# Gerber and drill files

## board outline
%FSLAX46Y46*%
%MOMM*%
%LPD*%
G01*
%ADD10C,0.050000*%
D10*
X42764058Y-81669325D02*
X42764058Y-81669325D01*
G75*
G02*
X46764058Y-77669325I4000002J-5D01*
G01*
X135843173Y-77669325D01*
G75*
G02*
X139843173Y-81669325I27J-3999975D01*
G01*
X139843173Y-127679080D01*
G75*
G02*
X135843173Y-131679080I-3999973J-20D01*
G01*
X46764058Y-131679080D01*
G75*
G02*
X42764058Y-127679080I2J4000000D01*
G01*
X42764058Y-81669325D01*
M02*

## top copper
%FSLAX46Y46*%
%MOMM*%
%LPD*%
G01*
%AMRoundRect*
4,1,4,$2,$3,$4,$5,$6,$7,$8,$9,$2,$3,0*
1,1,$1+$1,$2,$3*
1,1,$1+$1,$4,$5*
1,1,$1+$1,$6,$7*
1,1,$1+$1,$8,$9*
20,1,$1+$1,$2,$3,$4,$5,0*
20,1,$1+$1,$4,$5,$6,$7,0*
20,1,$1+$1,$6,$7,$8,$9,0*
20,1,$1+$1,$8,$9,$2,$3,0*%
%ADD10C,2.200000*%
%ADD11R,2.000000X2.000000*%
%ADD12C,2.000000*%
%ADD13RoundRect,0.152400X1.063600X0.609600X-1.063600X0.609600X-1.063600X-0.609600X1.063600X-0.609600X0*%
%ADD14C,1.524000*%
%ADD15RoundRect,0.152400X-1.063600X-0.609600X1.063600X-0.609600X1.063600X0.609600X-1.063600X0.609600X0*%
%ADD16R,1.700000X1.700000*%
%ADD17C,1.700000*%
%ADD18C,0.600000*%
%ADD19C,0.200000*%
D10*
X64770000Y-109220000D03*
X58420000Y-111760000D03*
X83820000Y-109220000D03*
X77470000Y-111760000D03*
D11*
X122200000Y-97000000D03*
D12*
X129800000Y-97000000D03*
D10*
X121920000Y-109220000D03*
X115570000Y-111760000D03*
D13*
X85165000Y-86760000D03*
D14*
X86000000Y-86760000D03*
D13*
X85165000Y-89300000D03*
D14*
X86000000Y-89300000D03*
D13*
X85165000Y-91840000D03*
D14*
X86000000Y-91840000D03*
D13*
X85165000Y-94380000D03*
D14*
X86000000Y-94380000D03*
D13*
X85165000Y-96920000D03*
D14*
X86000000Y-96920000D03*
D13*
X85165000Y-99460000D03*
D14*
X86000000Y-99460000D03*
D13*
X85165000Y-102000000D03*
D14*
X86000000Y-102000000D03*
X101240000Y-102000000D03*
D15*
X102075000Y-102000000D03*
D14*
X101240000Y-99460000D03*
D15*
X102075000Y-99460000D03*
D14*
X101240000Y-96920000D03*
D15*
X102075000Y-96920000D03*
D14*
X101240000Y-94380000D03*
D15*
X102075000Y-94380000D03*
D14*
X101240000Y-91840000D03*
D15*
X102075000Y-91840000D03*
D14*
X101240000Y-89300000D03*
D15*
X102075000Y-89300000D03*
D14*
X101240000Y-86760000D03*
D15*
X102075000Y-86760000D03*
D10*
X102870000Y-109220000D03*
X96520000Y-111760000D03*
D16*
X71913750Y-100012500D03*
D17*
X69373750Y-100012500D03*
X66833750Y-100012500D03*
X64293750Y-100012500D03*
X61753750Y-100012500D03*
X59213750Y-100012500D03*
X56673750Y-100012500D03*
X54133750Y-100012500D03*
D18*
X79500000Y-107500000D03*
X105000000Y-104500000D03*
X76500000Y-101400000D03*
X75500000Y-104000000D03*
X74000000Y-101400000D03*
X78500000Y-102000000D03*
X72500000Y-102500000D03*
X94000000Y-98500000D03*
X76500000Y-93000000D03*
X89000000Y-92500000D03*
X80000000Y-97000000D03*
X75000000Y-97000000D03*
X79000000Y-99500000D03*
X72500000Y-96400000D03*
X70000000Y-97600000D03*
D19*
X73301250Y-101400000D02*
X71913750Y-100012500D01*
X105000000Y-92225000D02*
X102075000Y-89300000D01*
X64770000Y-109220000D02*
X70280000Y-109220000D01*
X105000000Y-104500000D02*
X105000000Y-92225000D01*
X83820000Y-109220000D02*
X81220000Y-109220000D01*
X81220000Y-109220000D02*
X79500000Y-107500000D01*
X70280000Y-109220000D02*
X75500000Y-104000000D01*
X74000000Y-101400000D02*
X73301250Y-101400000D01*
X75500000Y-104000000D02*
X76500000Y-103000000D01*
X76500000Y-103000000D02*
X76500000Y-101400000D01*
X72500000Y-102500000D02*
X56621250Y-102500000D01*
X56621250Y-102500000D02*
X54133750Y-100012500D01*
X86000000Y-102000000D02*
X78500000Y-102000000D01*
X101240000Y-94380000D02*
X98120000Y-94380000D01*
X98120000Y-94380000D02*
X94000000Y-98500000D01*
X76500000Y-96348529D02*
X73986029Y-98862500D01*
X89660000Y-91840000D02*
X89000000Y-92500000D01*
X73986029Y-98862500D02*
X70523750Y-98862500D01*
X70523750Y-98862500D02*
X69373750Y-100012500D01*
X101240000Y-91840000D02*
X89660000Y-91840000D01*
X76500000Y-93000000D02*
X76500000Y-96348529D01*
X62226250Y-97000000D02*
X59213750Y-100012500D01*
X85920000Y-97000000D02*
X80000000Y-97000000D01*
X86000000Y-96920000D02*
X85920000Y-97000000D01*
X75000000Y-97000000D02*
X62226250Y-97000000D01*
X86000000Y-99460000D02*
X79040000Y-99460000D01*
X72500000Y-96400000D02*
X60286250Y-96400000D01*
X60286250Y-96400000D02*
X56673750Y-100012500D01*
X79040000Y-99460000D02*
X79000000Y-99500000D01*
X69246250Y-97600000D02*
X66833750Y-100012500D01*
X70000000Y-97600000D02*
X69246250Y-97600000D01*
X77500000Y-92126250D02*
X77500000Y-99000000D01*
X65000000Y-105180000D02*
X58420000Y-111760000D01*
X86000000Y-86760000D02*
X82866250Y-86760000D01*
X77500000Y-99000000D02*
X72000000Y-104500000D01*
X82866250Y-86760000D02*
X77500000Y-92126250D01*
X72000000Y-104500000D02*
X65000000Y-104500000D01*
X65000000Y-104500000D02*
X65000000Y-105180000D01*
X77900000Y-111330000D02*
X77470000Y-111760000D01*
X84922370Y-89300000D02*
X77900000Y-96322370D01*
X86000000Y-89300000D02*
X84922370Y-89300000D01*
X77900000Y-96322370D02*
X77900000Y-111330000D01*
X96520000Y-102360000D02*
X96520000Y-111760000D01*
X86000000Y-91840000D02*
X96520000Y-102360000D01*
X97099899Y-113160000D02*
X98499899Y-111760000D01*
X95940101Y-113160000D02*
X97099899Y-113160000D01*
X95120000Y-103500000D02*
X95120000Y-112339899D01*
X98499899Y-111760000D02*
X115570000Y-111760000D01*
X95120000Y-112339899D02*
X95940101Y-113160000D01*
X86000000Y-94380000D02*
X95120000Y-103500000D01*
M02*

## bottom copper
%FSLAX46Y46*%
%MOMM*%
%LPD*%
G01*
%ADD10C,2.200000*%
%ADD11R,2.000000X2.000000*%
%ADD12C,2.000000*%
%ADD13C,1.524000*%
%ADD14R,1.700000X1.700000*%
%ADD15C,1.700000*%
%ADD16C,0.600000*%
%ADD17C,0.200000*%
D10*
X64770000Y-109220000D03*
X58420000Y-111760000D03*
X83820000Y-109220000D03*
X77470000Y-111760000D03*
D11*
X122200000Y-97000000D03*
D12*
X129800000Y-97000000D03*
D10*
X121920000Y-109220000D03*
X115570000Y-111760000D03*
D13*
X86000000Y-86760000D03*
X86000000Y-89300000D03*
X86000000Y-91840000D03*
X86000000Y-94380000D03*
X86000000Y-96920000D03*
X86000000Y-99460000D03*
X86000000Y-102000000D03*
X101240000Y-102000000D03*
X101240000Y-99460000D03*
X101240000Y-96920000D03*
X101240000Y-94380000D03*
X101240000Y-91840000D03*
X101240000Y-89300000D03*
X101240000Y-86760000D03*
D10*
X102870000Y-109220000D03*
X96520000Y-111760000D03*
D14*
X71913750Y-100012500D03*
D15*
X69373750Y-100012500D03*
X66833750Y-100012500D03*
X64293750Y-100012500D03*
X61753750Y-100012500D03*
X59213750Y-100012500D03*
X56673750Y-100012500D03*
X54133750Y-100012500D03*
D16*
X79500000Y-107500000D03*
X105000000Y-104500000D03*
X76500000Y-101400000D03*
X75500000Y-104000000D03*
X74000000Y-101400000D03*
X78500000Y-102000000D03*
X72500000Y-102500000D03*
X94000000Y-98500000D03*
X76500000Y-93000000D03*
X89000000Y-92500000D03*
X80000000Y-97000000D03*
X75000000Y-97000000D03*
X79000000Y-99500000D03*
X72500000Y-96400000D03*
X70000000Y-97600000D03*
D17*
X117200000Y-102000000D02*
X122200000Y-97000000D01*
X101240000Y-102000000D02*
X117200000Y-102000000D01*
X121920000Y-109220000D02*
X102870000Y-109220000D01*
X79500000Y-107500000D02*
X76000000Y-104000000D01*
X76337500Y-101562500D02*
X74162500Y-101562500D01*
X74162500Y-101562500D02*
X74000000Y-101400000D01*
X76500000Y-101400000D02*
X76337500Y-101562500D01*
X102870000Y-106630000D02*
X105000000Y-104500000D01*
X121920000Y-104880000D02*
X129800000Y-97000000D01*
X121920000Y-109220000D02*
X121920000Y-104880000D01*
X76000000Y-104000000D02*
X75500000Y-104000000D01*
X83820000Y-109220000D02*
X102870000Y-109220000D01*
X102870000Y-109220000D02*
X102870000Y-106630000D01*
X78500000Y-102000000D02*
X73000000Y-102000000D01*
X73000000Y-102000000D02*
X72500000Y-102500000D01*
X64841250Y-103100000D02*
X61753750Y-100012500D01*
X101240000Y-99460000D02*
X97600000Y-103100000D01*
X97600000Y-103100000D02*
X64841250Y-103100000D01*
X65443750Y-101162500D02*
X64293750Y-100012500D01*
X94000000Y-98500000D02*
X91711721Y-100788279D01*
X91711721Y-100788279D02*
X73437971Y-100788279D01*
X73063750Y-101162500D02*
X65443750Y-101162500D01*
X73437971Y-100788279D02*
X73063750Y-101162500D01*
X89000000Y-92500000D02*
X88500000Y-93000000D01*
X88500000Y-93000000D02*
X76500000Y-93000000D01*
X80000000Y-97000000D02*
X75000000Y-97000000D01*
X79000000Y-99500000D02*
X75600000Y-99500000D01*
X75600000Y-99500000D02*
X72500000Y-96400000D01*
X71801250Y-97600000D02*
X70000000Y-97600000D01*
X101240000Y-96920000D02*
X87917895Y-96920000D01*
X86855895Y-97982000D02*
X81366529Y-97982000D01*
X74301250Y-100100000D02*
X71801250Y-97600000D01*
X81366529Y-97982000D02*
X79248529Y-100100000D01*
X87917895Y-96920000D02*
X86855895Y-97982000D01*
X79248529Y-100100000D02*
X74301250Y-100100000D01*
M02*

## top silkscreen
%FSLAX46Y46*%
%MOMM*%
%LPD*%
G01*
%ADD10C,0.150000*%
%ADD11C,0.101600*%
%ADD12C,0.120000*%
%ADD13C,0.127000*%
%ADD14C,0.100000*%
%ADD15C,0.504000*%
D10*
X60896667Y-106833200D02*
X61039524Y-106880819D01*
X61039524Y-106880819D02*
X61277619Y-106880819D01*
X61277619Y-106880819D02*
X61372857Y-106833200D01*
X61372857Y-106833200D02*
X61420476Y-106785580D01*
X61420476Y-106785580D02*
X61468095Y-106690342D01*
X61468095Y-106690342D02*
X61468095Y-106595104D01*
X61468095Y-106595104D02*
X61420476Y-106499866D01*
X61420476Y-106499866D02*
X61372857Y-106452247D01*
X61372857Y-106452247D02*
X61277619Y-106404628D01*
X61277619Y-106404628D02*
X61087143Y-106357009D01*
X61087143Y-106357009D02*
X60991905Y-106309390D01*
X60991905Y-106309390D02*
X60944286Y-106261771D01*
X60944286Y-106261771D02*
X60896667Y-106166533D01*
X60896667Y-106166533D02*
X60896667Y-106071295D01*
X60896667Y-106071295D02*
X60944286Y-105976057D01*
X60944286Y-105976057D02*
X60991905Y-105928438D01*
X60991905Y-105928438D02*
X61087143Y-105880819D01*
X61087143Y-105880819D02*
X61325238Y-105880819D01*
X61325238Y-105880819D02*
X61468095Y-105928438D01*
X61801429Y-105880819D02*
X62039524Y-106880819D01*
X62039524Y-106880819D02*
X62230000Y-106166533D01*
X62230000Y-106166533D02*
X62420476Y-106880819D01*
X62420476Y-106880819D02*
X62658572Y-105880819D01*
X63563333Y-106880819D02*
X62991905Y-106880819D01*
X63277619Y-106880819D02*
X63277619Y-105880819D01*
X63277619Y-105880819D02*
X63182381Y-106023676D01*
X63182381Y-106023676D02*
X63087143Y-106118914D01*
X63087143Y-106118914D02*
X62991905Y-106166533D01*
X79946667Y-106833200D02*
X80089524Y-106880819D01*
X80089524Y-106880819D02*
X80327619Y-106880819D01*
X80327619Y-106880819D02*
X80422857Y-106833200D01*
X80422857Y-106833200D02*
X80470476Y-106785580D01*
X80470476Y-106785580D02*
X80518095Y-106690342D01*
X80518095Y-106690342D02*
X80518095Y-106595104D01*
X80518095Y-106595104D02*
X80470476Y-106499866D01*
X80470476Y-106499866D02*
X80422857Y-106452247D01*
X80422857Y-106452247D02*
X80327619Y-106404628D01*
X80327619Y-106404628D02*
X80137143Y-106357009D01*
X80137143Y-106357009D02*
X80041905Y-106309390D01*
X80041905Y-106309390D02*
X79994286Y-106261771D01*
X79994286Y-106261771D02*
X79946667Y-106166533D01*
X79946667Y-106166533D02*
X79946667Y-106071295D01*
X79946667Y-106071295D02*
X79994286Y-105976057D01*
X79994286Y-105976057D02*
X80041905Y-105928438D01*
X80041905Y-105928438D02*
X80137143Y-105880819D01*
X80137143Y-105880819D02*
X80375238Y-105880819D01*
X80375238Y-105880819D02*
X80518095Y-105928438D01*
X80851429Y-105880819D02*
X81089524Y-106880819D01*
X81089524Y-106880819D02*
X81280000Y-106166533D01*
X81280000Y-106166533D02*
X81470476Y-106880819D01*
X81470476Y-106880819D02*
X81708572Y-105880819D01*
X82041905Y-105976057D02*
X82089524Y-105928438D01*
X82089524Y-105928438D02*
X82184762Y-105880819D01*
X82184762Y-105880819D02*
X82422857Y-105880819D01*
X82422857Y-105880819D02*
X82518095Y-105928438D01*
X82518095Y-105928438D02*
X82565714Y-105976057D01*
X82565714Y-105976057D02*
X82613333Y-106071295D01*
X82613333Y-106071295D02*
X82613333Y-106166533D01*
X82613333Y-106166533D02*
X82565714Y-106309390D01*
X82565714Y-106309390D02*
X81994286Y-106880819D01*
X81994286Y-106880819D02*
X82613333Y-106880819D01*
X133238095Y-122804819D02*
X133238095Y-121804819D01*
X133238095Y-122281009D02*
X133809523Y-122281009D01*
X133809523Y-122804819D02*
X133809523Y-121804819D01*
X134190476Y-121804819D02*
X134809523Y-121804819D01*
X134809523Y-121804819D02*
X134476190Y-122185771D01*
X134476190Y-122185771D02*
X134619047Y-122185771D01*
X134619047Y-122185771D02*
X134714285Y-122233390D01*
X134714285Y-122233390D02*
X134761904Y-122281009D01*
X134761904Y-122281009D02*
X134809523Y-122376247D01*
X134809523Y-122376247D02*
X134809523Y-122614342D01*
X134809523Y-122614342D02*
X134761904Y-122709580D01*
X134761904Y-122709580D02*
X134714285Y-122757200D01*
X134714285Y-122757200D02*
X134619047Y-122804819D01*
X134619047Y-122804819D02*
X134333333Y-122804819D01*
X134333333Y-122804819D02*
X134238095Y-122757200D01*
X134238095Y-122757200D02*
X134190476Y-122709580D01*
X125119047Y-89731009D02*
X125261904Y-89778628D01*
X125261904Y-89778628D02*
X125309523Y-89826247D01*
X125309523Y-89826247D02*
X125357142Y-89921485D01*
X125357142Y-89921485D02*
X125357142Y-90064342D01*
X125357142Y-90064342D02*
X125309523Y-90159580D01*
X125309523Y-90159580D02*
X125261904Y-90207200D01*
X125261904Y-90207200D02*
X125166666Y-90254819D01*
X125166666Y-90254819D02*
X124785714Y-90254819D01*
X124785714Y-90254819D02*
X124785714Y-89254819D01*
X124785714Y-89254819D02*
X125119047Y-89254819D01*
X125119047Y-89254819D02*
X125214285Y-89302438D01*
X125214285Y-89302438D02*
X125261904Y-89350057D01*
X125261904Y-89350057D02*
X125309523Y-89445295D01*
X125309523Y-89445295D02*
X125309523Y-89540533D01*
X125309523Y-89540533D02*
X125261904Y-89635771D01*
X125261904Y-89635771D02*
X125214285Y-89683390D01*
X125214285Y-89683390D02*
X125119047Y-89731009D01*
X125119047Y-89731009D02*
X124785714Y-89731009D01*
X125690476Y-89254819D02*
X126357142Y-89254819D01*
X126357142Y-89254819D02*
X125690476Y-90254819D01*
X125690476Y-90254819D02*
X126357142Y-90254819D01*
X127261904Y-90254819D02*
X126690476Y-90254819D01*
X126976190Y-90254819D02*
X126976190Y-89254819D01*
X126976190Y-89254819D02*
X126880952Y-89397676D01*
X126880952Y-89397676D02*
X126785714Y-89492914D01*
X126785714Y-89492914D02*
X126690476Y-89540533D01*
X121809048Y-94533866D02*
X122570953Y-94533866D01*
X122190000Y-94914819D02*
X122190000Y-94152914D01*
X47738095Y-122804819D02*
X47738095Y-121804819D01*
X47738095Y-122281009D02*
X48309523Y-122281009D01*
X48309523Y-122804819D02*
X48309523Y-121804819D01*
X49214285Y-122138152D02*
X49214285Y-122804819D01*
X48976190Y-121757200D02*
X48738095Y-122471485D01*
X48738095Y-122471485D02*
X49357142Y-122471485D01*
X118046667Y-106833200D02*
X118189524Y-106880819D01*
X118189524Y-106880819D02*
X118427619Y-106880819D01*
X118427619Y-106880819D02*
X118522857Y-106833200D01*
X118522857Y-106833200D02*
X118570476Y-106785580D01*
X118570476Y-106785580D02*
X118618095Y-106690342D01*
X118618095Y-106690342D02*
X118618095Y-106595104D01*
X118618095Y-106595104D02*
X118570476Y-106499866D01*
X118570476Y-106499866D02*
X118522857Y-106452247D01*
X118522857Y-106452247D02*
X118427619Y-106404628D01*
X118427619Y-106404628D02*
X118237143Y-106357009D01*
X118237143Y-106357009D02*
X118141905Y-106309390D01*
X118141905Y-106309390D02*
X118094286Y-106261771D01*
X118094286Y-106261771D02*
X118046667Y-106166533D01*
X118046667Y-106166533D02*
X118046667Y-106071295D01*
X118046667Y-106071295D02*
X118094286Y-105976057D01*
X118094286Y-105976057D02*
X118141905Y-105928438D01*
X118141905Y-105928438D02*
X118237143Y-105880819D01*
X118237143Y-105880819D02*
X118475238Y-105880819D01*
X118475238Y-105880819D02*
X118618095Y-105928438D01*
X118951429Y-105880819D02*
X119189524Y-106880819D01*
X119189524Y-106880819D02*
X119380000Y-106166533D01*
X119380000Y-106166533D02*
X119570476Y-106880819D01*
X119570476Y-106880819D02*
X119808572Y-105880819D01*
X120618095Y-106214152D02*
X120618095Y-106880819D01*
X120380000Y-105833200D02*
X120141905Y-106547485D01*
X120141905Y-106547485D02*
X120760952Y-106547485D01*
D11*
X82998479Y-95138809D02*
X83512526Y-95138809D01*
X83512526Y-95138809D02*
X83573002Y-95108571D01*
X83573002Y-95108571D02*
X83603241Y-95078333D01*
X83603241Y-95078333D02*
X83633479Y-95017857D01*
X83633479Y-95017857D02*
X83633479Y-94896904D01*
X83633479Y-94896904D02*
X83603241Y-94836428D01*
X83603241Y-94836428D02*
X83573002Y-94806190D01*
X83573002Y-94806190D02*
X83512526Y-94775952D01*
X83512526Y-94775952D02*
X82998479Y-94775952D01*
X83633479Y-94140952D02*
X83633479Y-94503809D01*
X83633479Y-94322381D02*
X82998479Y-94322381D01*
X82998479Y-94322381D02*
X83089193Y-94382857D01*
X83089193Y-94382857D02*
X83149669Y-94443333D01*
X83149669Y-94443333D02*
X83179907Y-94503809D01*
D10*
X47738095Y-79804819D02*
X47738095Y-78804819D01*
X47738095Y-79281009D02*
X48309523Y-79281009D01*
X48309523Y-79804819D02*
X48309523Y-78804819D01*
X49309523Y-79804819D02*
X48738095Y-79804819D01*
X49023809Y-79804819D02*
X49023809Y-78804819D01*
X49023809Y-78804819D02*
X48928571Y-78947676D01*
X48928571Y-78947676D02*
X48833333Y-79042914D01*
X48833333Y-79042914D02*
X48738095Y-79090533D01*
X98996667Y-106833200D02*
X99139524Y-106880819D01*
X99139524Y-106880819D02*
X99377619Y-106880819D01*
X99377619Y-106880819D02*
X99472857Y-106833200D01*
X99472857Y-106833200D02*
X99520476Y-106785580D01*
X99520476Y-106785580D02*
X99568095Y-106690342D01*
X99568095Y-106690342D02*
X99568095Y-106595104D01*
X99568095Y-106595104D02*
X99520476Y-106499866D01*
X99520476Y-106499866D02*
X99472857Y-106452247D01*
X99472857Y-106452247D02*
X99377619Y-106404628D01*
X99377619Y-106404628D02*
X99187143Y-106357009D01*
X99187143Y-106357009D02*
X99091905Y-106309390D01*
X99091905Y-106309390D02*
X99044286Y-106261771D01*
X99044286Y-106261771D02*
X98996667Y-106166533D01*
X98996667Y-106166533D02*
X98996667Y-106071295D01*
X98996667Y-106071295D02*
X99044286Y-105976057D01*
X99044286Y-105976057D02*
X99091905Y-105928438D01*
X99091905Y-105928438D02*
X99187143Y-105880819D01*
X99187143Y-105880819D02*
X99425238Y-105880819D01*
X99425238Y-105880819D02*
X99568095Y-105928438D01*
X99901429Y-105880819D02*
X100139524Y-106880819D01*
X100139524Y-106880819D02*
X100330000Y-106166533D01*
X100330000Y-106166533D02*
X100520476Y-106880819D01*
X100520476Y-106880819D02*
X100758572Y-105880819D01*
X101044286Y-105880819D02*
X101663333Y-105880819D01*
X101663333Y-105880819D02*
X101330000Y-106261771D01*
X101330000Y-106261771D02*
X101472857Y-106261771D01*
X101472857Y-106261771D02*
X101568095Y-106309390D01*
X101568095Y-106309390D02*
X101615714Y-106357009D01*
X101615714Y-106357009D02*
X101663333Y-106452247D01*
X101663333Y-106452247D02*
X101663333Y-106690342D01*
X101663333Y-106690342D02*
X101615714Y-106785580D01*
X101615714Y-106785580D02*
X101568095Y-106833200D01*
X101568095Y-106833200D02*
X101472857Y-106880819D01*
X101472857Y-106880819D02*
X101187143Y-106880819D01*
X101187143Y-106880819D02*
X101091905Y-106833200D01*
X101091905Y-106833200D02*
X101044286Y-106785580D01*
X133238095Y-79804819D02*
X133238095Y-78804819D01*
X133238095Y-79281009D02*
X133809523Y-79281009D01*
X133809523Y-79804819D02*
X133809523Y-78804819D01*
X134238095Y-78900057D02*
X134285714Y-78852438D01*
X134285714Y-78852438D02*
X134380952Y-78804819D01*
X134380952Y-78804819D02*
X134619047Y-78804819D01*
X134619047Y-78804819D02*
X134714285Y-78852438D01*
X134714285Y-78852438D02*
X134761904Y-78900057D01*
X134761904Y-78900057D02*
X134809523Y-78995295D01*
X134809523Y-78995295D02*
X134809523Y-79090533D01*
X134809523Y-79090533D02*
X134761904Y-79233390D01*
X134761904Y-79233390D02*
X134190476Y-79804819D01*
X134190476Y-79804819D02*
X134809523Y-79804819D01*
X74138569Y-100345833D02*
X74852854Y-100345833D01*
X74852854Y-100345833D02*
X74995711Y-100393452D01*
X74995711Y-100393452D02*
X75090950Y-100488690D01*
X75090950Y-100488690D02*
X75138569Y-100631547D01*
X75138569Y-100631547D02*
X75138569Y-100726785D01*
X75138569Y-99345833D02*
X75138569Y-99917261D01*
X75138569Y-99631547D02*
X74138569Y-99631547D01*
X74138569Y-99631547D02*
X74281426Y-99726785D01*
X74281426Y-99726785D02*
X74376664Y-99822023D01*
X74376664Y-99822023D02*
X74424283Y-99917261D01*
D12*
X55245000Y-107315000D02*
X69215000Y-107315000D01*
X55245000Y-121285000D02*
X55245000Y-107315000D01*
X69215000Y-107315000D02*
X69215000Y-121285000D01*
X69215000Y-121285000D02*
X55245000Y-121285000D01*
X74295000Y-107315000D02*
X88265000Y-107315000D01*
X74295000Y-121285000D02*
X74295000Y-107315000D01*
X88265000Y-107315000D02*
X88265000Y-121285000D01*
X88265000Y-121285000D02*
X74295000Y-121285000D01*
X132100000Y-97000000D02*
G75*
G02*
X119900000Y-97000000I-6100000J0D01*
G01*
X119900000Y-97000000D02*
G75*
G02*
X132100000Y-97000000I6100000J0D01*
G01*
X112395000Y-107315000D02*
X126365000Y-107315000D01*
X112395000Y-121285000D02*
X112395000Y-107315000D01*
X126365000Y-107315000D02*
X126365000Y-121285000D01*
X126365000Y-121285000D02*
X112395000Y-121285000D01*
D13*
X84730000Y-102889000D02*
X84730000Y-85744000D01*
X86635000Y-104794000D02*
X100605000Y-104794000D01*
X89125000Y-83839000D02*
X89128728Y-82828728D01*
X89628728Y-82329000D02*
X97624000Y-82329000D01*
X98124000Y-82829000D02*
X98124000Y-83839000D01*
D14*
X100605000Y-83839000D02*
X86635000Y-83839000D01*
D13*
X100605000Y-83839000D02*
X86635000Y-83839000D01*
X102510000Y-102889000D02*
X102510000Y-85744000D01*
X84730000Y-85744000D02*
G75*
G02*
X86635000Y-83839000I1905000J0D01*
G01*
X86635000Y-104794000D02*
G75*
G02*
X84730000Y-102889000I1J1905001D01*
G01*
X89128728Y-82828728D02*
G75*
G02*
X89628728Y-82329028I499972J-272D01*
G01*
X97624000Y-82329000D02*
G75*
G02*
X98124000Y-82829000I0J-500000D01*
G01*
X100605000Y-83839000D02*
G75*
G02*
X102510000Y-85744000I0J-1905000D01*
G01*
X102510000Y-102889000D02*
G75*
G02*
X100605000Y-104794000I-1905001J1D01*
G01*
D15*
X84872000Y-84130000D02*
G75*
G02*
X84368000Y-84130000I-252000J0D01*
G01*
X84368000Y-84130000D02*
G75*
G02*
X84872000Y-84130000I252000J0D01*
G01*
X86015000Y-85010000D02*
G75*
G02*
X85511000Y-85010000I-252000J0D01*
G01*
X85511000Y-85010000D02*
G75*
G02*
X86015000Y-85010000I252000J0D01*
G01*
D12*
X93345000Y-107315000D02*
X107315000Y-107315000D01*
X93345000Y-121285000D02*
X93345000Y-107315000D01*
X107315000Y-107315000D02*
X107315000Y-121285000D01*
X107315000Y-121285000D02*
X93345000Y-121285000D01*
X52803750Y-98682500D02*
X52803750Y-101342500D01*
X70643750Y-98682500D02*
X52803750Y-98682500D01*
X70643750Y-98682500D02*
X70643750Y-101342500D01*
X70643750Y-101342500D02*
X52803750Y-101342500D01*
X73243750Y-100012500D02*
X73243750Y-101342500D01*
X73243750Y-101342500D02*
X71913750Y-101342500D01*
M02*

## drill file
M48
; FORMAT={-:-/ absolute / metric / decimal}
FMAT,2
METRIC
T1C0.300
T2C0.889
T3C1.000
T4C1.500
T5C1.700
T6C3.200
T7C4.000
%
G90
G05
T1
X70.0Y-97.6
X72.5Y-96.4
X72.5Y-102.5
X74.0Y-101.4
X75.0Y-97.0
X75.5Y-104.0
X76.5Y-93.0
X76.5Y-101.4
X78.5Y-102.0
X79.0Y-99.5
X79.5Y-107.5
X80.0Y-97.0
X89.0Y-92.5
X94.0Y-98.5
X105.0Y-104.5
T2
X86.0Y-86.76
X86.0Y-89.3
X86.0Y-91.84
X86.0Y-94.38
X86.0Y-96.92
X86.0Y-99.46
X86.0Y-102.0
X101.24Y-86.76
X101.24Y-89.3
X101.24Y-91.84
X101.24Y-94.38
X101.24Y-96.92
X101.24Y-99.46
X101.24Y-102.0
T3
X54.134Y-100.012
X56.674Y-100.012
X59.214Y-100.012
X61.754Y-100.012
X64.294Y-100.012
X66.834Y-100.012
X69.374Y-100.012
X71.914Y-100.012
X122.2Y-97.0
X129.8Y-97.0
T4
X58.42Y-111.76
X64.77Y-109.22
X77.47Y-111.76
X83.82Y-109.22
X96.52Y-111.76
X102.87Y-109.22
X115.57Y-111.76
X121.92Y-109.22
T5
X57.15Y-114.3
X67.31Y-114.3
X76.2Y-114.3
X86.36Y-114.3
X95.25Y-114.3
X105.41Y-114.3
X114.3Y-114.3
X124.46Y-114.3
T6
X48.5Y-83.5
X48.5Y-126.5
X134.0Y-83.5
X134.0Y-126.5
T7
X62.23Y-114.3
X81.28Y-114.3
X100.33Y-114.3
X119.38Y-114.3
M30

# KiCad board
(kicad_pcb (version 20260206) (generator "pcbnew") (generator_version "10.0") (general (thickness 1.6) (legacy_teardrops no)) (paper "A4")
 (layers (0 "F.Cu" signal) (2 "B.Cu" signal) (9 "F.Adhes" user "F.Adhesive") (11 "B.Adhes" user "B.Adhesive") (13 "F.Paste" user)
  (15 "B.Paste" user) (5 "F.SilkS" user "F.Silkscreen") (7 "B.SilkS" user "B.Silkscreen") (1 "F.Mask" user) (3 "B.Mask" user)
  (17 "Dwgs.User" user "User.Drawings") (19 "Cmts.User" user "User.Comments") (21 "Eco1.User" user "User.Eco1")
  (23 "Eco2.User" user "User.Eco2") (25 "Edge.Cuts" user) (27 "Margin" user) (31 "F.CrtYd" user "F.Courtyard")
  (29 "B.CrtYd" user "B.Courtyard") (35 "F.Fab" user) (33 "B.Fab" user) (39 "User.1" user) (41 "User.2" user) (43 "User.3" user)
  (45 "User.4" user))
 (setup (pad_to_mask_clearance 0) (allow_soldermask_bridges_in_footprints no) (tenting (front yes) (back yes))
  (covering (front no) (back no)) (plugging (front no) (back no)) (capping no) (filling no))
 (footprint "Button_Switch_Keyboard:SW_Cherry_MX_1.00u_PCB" (layer "F.Cu") (at 64.77 109.22)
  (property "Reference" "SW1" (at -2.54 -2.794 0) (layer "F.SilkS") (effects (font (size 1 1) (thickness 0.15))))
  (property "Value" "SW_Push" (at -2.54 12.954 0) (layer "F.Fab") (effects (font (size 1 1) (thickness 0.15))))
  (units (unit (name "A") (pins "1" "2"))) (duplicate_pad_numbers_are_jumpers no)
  (fp_line (start -9.525 -1.905) (end 4.445 -1.905) (stroke (width 0.12) (type solid)) (layer "F.SilkS"))
  (fp_line (start -9.525 12.065) (end -9.525 -1.905) (stroke (width 0.12) (type solid)) (layer "F.SilkS"))
  (fp_line (start 4.445 -1.905) (end 4.445 12.065) (stroke (width 0.12) (type solid)) (layer "F.SilkS"))
  (fp_line (start 4.445 12.065) (end -9.525 12.065) (stroke (width 0.12) (type solid)) (layer "F.SilkS"))
  (pad "" np_thru_hole circle (at -7.62 5.08) (size 1.7 1.7) (drill 1.7) (layers "*.Cu" "*.Mask"))
  (pad "" np_thru_hole circle (at -2.54 5.08) (size 4 4) (drill 4) (layers "*.Cu" "*.Mask"))
  (pad "" np_thru_hole circle (at 2.54 5.08) (size 1.7 1.7) (drill 1.7) (layers "*.Cu" "*.Mask"))
  (pad "1" thru_hole circle (at 0 0) (size 2.2 2.2) (drill 1.5) (layers "*.Cu" "*.Mask") (remove_unused_layers no) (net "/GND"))
  (pad "2" thru_hole circle (at -6.35 2.54) (size 2.2 2.2) (drill 1.5) (layers "*.Cu" "*.Mask") (remove_unused_layers no)
   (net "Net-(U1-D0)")))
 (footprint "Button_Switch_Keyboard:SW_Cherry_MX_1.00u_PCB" (layer "F.Cu") (at 83.82 109.22)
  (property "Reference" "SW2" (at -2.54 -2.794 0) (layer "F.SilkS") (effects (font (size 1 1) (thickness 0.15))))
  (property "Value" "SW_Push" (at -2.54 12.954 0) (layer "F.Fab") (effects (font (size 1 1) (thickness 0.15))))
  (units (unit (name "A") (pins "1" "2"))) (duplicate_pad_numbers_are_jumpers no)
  (fp_line (start -9.525 -1.905) (end 4.445 -1.905) (stroke (width 0.12) (type solid)) (layer "F.SilkS"))
  (fp_line (start -9.525 12.065) (end -9.525 -1.905) (stroke (width 0.12) (type solid)) (layer "F.SilkS"))
  (fp_line (start 4.445 -1.905) (end 4.445 12.065) (stroke (width 0.12) (type solid)) (layer "F.SilkS"))
  (fp_line (start 4.445 12.065) (end -9.525 12.065) (stroke (width 0.12) (type solid)) (layer "F.SilkS"))
  (pad "" np_thru_hole circle (at -7.62 5.08) (size 1.7 1.7) (drill 1.7) (layers "*.Cu" "*.Mask"))
  (pad "" np_thru_hole circle (at -2.54 5.08) (size 4 4) (drill 4) (layers "*.Cu" "*.Mask"))
  (pad "" np_thru_hole circle (at 2.54 5.08) (size 1.7 1.7) (drill 1.7) (layers "*.Cu" "*.Mask"))
  (pad "1" thru_hole circle (at 0 0) (size 2.2 2.2) (drill 1.5) (layers "*.Cu" "*.Mask") (remove_unused_layers no) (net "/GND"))
  (pad "2" thru_hole circle (at -6.35 2.54) (size 2.2 2.2) (drill 1.5) (layers "*.Cu" "*.Mask") (remove_unused_layers no)
   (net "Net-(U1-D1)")))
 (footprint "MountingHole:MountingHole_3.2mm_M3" (layer "F.Cu") (at 134 126.5)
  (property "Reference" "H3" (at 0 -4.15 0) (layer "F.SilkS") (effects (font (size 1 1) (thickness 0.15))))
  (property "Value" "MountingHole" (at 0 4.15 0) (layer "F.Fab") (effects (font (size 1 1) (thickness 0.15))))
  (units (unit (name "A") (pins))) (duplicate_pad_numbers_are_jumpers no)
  (pad "" np_thru_hole circle (at 0 0) (size 3.2 3.2) (drill 3.2) (layers "*.Cu" "*.Mask")))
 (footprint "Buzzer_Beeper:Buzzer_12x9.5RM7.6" (layer "F.Cu") (at 122.2 97)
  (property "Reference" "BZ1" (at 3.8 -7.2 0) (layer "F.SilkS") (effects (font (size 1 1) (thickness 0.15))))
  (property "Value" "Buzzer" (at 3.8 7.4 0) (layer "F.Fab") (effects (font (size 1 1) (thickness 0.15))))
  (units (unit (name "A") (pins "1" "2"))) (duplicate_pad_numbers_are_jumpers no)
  (fp_circle (center 3.8 0) (end 9.9 0) (stroke (width 0.12) (type solid)) (fill no) (layer "F.SilkS"))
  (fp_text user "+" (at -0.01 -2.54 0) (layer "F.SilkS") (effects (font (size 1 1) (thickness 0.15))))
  (pad "1" thru_hole rect (at 0 0) (size 2 2) (drill 1) (layers "*.Cu" "*.Mask") (remove_unused_layers no) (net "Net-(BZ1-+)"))
  (pad "2" thru_hole circle (at 7.6 0) (size 2 2) (drill 1) (layers "*.Cu" "*.Mask") (remove_unused_layers no) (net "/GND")))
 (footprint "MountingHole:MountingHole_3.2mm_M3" (layer "F.Cu") (at 48.5 126.5)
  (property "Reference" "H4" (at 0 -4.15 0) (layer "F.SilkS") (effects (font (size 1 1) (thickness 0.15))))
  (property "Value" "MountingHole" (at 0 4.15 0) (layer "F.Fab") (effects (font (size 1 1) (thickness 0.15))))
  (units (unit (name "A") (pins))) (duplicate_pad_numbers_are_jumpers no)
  (pad "" np_thru_hole circle (at 0 0) (size 3.2 3.2) (drill 3.2) (layers "*.Cu" "*.Mask")))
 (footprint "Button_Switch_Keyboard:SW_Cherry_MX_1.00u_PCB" (layer "F.Cu") (at 121.92 109.22)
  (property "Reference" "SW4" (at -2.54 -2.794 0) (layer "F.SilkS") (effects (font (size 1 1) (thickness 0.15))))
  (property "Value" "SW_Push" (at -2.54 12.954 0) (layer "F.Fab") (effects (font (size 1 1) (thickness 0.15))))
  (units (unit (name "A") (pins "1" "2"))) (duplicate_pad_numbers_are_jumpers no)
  (fp_line (start -9.525 -1.905) (end 4.445 -1.905) (stroke (width 0.12) (type solid)) (layer "F.SilkS"))
  (fp_line (start -9.525 12.065) (end -9.525 -1.905) (stroke (width 0.12) (type solid)) (layer "F.SilkS"))
  (fp_line (start 4.445 -1.905) (end 4.445 12.065) (stroke (width 0.12) (type solid)) (layer "F.SilkS"))
  (fp_line (start 4.445 12.065) (end -9.525 12.065) (stroke (width 0.12) (type solid)) (layer "F.SilkS"))
  (pad "" np_thru_hole circle (at -7.62 5.08) (size 1.7 1.7) (drill 1.7) (layers "*.Cu" "*.Mask"))
  (pad "" np_thru_hole circle (at -2.54 5.08) (size 4 4) (drill 4) (layers "*.Cu" "*.Mask"))
  (pad "" np_thru_hole circle (at 2.54 5.08) (size 1.7 1.7) (drill 1.7) (layers "*.Cu" "*.Mask"))
  (pad "1" thru_hole circle (at 0 0) (size 2.2 2.2) (drill 1.5) (layers "*.Cu" "*.Mask") (remove_unused_layers no) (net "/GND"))
  (pad "2" thru_hole circle (at -6.35 2.54) (size 2.2 2.2) (drill 1.5) (layers "*.Cu" "*.Mask") (remove_unused_layers no)
   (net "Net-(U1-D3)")))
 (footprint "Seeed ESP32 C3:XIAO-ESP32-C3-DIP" (layer "F.Cu") (at 93.62 94.38 90)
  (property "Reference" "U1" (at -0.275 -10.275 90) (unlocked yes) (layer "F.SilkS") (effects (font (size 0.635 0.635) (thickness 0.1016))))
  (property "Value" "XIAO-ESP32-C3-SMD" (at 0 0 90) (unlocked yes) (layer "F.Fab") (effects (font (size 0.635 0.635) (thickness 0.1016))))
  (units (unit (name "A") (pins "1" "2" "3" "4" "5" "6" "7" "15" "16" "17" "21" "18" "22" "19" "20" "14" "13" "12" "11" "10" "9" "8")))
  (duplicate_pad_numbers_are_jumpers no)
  (fp_line (start -8.509 -8.89) (end 8.636 -8.89) (stroke (width 0.127) (type solid)) (layer "F.SilkS"))
  (fp_line (start -10.414 -6.985) (end -10.414 6.985) (stroke (width 0.127) (type solid)) (layer "F.SilkS"))
  (fp_line (start 10.541 -4.495) (end 11.551272 -4.491272) (stroke (width 0.127) (type solid)) (layer "F.SilkS"))
  (fp_line (start 12.051 -3.991272) (end 12.051 4.004) (stroke (width 0.127) (type solid)) (layer "F.SilkS"))
  (fp_line (start 11.551 4.504) (end 10.541 4.504) (stroke (width 0.127) (type solid)) (layer "F.SilkS"))
  (fp_line (start 10.541 6.985) (end 10.541 -6.985) (stroke (width 0.1) (type solid)) (layer "F.SilkS"))
  (fp_line (start 10.541 6.985) (end 10.541 -6.985) (stroke (width 0.127) (type solid)) (layer "F.SilkS"))
  (fp_line (start -8.509 8.89) (end 8.636 8.89) (stroke (width 0.127) (type solid)) (layer "F.SilkS"))
  (fp_arc (start 8.636 -8.89) (mid 9.983038 -8.332038) (end 10.541 -6.985) (stroke (width 0.127) (type solid)) (layer "F.SilkS"))
  (fp_arc (start -10.414 -6.985) (mid -9.856038 -8.332038) (end -8.509 -8.89) (stroke (width 0.127) (type solid)) (layer "F.SilkS"))
  (fp_arc (start 11.551272 -4.491272) (mid 11.904644 -4.344724) (end 12.051 -3.991272) (stroke (width 0.127) (type default))
   (layer "F.SilkS"))
  (fp_arc (start 12.051 4.004) (mid 11.904553 4.357553) (end 11.551 4.504) (stroke (width 0.127) (type default)) (layer "F.SilkS"))
  (fp_arc (start 10.541 6.985) (mid 9.983038 8.332038) (end 8.636 8.89) (stroke (width 0.127) (type solid)) (layer "F.SilkS"))
  (fp_arc (start -8.509 8.89) (mid -9.856038 8.332038) (end -10.414 6.985) (stroke (width 0.127) (type solid)) (layer "F.SilkS"))
  (fp_circle (center 10.25 -9) (end 10.504 -9) (stroke (width 0.5) (type solid)) (fill yes) (layer "F.SilkS"))
  (fp_circle (center 9.37 -7.857) (end 9.624 -7.857) (stroke (width 0.5) (type solid)) (fill yes) (layer "F.SilkS"))
  (pad "1" smd roundrect (at 7.62 -8.455 180) (size 2.432 1.524) (layers "F.Cu" "F.Mask") (roundrect_rratio 0.1) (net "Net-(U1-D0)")
   (thermal_bridge_angle 45))
  (pad "1" thru_hole circle (at 7.62 -7.62 180) (size 1.524 1.524) (drill 0.889) (layers "*.Cu" "*.Mask") (remove_unused_layers no)
   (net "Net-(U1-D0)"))
  (pad "2" smd roundrect (at 5.08 -8.455 180) (size 2.432 1.524) (layers "F.Cu" "F.Mask") (roundrect_rratio 0.1) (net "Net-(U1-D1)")
   (thermal_bridge_angle 45))
  (pad "2" thru_hole circle (at 5.08 -7.62 180) (size 1.524 1.524) (drill 0.889) (layers "*.Cu" "*.Mask") (remove_unused_layers no)
   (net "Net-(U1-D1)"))
  (pad "3" smd roundrect (at 2.54 -8.455 180) (size 2.432 1.524) (layers "F.Cu" "F.Mask") (roundrect_rratio 0.1) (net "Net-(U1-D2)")
   (thermal_bridge_angle 45))
  (pad "3" thru_hole circle (at 2.54 -7.62 180) (size 1.524 1.524) (drill 0.889) (layers "*.Cu" "*.Mask") (remove_unused_layers no)
   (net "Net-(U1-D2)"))
  (pad "4" smd roundrect (at 0 -8.455 180) (size 2.432 1.524) (layers "F.Cu" "F.Mask") (roundrect_rratio 0.1) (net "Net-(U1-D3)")
   (thermal_bridge_angle 45))
  (pad "4" thru_hole circle (at 0 -7.62 180) (size 1.524 1.524) (drill 0.889) (layers "*.Cu" "*.Mask") (remove_unused_layers no)
   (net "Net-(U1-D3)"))
  (pad "5" smd roundrect (at -2.54 -8.455 180) (size 2.432 1.524) (layers "F.Cu" "F.Mask") (roundrect_rratio 0.1) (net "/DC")
   (thermal_bridge_angle 45))
  (pad "5" thru_hole circle (at -2.54 -7.62 180) (size 1.524 1.524) (drill 0.889) (layers "*.Cu" "*.Mask") (remove_unused_layers no)
   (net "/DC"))
  (pad "6" smd roundrect (at -5.08 -8.455 180) (size 2.432 1.524) (layers "F.Cu" "F.Mask") (roundrect_rratio 0.1) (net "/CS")
   (thermal_bridge_angle 45))
  (pad "6" thru_hole circle (at -5.08 -7.62 180) (size 1.524 1.524) (drill 0.889) (layers "*.Cu" "*.Mask") (remove_unused_layers no)
   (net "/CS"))
  (pad "7" smd roundrect (at -7.62 -8.455 180) (size 2.432 1.524) (layers "F.Cu" "F.Mask") (roundrect_rratio 0.1) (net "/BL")
   (thermal_bridge_angle 45))
  (pad "7" thru_hole circle (at -7.62 -7.62 180) (size 1.524 1.524) (drill 0.889) (layers "*.Cu" "*.Mask") (remove_unused_layers no)
   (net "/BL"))
  (pad "8" thru_hole circle (at -7.62 7.62) (size 1.524 1.524) (drill 0.889) (layers "*.Cu" "*.Mask") (remove_unused_layers no)
   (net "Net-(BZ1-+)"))
  (pad "8" smd roundrect (at -7.62 8.455) (size 2.432 1.524) (layers "F.Cu" "F.Mask") (roundrect_rratio 0.1) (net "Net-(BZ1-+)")
   (thermal_bridge_angle 45))
  (pad "9" thru_hole circle (at -5.08 7.62) (size 1.524 1.524) (drill 0.889) (layers "*.Cu" "*.Mask") (remove_unused_layers no) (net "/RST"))
  (pad "9" smd roundrect (at -5.08 8.455) (size 2.432 1.524) (layers "F.Cu" "F.Mask") (roundrect_rratio 0.1) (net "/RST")
   (thermal_bridge_angle 45))
  (pad "10" thru_hole circle (at -2.54 7.62) (size 1.524 1.524) (drill 0.889) (layers "*.Cu" "*.Mask") (remove_unused_layers no)
   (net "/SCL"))
  (pad "10" smd roundrect (at -2.54 8.455) (size 2.432 1.524) (layers "F.Cu" "F.Mask") (roundrect_rratio 0.1) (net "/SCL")
   (thermal_bridge_angle 45))
  (pad "11" thru_hole circle (at 0 7.62) (size 1.524 1.524) (drill 0.889) (layers "*.Cu" "*.Mask") (remove_unused_layers no) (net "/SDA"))
  (pad "11" smd roundrect (at 0 8.455) (size 2.432 1.524) (layers "F.Cu" "F.Mask") (roundrect_rratio 0.1) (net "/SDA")
   (thermal_bridge_angle 45))
  (pad "12" thru_hole circle (at 2.54 7.62) (size 1.524 1.524) (drill 0.889) (layers "*.Cu" "*.Mask") (remove_unused_layers no)
   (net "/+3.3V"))
  (pad "12" smd roundrect (at 2.54 8.455) (size 2.432 1.524) (layers "F.Cu" "F.Mask") (roundrect_rratio 0.1) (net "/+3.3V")
   (thermal_bridge_angle 45))
  (pad "13" thru_hole circle (at 5.08 7.62) (size 1.524 1.524) (drill 0.889) (layers "*.Cu" "*.Mask") (remove_unused_layers no) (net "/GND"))
  (pad "13" smd roundrect (at 5.08 8.455) (size 2.432 1.524) (layers "F.Cu" "F.Mask") (roundrect_rratio 0.1) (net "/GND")
   (thermal_bridge_angle 45))
  (pad "14" thru_hole circle (at 7.62 7.62) (size 1.524 1.524) (drill 0.889) (layers "*.Cu" "*.Mask") (remove_unused_layers no)
   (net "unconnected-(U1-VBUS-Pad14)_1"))
  (pad "14" smd roundrect (at 7.62 8.455) (size 2.432 1.524) (layers "F.Cu" "F.Mask") (roundrect_rratio 0.1)
   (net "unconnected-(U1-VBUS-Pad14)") (thermal_bridge_angle 45)))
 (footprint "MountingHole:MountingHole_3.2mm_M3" (layer "F.Cu") (at 48.5 83.5)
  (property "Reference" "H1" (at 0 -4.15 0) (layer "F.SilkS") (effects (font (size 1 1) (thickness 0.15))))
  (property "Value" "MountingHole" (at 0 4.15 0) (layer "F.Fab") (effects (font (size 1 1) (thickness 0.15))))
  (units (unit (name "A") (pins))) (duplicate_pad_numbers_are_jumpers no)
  (pad "" np_thru_hole circle (at 0 0) (size 3.2 3.2) (drill 3.2) (layers "*.Cu" "*.Mask")))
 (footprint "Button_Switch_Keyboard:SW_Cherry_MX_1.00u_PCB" (layer "F.Cu") (at 102.87 109.22)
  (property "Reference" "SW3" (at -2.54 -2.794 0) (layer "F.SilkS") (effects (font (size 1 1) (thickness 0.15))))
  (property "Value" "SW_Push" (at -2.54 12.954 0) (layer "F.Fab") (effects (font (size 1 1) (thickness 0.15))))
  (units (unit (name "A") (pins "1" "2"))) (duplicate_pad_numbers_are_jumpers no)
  (fp_line (start -9.525 -1.905) (end 4.445 -1.905) (stroke (width 0.12) (type solid)) (layer "F.SilkS"))
  (fp_line (start -9.525 12.065) (end -9.525 -1.905) (stroke (width 0.12) (type solid)) (layer "F.SilkS"))
  (fp_line (start 4.445 -1.905) (end 4.445 12.065) (stroke (width 0.12) (type solid)) (layer "F.SilkS"))
  (fp_line (start 4.445 12.065) (end -9.525 12.065) (stroke (width 0.12) (type solid)) (layer "F.SilkS"))
  (pad "" np_thru_hole circle (at -7.62 5.08) (size 1.7 1.7) (drill 1.7) (layers "*.Cu" "*.Mask"))
  (pad "" np_thru_hole circle (at -2.54 5.08) (size 4 4) (drill 4) (layers "*.Cu" "*.Mask"))
  (pad "" np_thru_hole circle (at 2.54 5.08) (size 1.7 1.7) (drill 1.7) (layers "*.Cu" "*.Mask"))
  (pad "1" thru_hole circle (at 0 0) (size 2.2 2.2) (drill 1.5) (layers "*.Cu" "*.Mask") (remove_unused_layers no) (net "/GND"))
  (pad "2" thru_hole circle (at -6.35 2.54) (size 2.2 2.2) (drill 1.5) (layers "*.Cu" "*.Mask") (remove_unused_layers no)
   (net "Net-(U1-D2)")))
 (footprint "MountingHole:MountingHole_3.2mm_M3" (layer "F.Cu") (at 134 83.5)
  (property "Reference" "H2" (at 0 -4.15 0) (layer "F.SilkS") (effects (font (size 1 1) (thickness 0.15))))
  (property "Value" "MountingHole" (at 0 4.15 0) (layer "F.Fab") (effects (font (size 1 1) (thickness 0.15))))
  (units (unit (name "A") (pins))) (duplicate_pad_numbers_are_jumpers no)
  (pad "" np_thru_hole circle (at 0 0) (size 3.2 3.2) (drill 3.2) (layers "*.Cu" "*.Mask")))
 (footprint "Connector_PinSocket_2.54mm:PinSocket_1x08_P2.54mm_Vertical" (layer "F.Cu") (at 71.91375 100.0125 -90)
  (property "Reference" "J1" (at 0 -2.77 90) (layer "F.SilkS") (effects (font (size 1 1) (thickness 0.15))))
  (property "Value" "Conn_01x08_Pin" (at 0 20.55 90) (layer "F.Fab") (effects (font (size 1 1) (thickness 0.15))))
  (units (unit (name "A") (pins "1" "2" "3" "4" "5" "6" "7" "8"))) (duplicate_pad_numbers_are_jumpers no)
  (fp_line (start -1.33 19.11) (end 1.33 19.11) (stroke (width 0.12) (type solid)) (layer "F.SilkS"))
  (fp_line (start -1.33 1.27) (end -1.33 19.11) (stroke (width 0.12) (type solid)) (layer "F.SilkS"))
  (fp_line (start -1.33 1.27) (end 1.33 1.27) (stroke (width 0.12) (type solid)) (layer "F.SilkS"))
  (fp_line (start 1.33 1.27) (end 1.33 19.11) (stroke (width 0.12) (type solid)) (layer "F.SilkS"))
  (fp_line (start 0 -1.33) (end 1.33 -1.33) (stroke (width 0.12) (type solid)) (layer "F.SilkS"))
  (fp_line (start 1.33 -1.33) (end 1.33 0) (stroke (width 0.12) (type solid)) (layer "F.SilkS"))
  (pad "1" thru_hole rect (at 0 0 270) (size 1.7 1.7) (drill 1) (layers "*.Cu" "*.Mask") (remove_unused_layers no) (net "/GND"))
  (pad "2" thru_hole circle (at 0 2.54 270) (size 1.7 1.7) (drill 1) (layers "*.Cu" "*.Mask") (remove_unused_layers no) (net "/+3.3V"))
  (pad "3" thru_hole circle (at 0 5.08 270) (size 1.7 1.7) (drill 1) (layers "*.Cu" "*.Mask") (remove_unused_layers no) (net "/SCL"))
  (pad "4" thru_hole circle (at 0 7.62 270) (size 1.7 1.7) (drill 1) (layers "*.Cu" "*.Mask") (remove_unused_layers no) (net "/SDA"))
  (pad "5" thru_hole circle (at 0 10.16 270) (size 1.7 1.7) (drill 1) (layers "*.Cu" "*.Mask") (remove_unused_layers no) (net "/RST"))
  (pad "6" thru_hole circle (at 0 12.7 270) (size 1.7 1.7) (drill 1) (layers "*.Cu" "*.Mask") (remove_unused_layers no) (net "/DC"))
  (pad "7" thru_hole circle (at 0 15.24 270) (size 1.7 1.7) (drill 1) (layers "*.Cu" "*.Mask") (remove_unused_layers no) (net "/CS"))
  (pad "8" thru_hole circle (at 0 17.78 270) (size 1.7 1.7) (drill 1) (layers "*.Cu" "*.Mask") (remove_unused_layers no) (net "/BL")))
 (gr_rect (start 42.764058 77.669325) (end 139.843173 131.67908) (radius 4) (stroke (width 0.05) (type default)) (fill no)
  (layer "Edge.Cuts"))
 (segment (start 117.2 102) (end 122.2 97) (width 0.2) (layer "B.Cu") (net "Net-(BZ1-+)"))
 (segment (start 101.24 102) (end 117.2 102) (width 0.2) (layer "B.Cu") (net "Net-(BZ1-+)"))
 (segment (start 73.30125 101.4) (end 71.91375 100.0125) (width 0.2) (layer "F.Cu") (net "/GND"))
 (segment (start 105 92.225) (end 102.075 89.3) (width 0.2) (layer "F.Cu") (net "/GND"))
 (segment (start 64.77 109.22) (end 70.28 109.22) (width 0.2) (layer "F.Cu") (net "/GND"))
 (segment (start 105 104.5) (end 105 92.225) (width 0.2) (layer "F.Cu") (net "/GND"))
 (segment (start 83.82 109.22) (end 81.22 109.22) (width 0.2) (layer "F.Cu") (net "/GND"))
 (segment (start 81.22 109.22) (end 79.5 107.5) (width 0.2) (layer "F.Cu") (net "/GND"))
 (segment (start 70.28 109.22) (end 75.5 104) (width 0.2) (layer "F.Cu") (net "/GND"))
 (segment (start 74 101.4) (end 73.30125 101.4) (width 0.2) (layer "F.Cu") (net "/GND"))
 (segment (start 75.5 104) (end 76.5 103) (width 0.2) (layer "F.Cu") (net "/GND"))
 (segment (start 76.5 103) (end 76.5 101.4) (width 0.2) (layer "F.Cu") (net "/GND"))
 (via (at 79.5 107.5) (size 0.6) (drill 0.3) (layers "F.Cu" "B.Cu") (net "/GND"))
 (via (at 105 104.5) (size 0.6) (drill 0.3) (layers "F.Cu" "B.Cu") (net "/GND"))
 (via (at 76.5 101.4) (size 0.6) (drill 0.3) (layers "F.Cu" "B.Cu") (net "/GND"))
 (via (at 75.5 104) (size 0.6) (drill 0.3) (layers "F.Cu" "B.Cu") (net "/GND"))
 (via (at 74 101.4) (size 0.6) (drill 0.3) (layers "F.Cu" "B.Cu") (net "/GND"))
 (segment (start 121.92 109.22) (end 102.87 109.22) (width 0.2) (layer "B.Cu") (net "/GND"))
 (segment (start 79.5 107.5) (end 76 104) (width 0.2) (layer "B.Cu") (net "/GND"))
 (segment (start 76.3375 101.5625) (end 74.1625 101.5625) (width 0.2) (layer "B.Cu") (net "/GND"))
 (segment (start 74.1625 101.5625) (end 74 101.4) (width 0.2) (layer "B.Cu") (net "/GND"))
 (segment (start 76.5 101.4) (end 76.3375 101.5625) (width 0.2) (layer "B.Cu") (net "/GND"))
 (segment (start 102.87 106.63) (end 105 104.5) (width 0.2) (layer "B.Cu") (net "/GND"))
 (segment (start 121.92 104.88) (end 129.8 97) (width 0.2) (layer "B.Cu") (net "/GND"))
 (segment (start 121.92 109.22) (end 121.92 104.88) (width 0.2) (layer "B.Cu") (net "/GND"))
 (segment (start 76 104) (end 75.5 104) (width 0.2) (layer "B.Cu") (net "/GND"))
 (segment (start 83.82 109.22) (end 102.87 109.22) (width 0.2) (layer "B.Cu") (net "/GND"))
 (segment (start 102.87 109.22) (end 102.87 106.63) (width 0.2) (layer "B.Cu") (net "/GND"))
 (segment (start 72.5 102.5) (end 56.62125 102.5) (width 0.2) (layer "F.Cu") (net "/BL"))
 (segment (start 56.62125 102.5) (end 54.13375 100.0125) (width 0.2) (layer "F.Cu") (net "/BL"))
 (segment (start 86 102) (end 78.5 102) (width 0.2) (layer "F.Cu") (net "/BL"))
 (via (at 78.5 102) (size 0.6) (drill 0.3) (layers "F.Cu" "B.Cu") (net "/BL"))
 (via (at 72.5 102.5) (size 0.6) (drill 0.3) (layers "F.Cu" "B.Cu") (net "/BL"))
 (segment (start 78.5 102) (end 73 102) (width 0.2) (layer "B.Cu") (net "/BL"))
 (segment (start 73 102) (end 72.5 102.5) (width 0.2) (layer "B.Cu") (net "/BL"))
 (segment (start 64.84125 103.1) (end 61.75375 100.0125) (width 0.2) (layer "B.Cu") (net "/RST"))
 (segment (start 101.24 99.46) (end 97.6 103.1) (width 0.2) (layer "B.Cu") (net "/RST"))
 (segment (start 97.6 103.1) (end 64.84125 103.1) (width 0.2) (layer "B.Cu") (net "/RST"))
 (segment (start 101.24 94.38) (end 98.12 94.38) (width 0.2) (layer "F.Cu") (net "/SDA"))
 (segment (start 98.12 94.38) (end 94 98.5) (width 0.2) (layer "F.Cu") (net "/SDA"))
 (via (at 94 98.5) (size 0.6) (drill 0.3) (layers "F.Cu" "B.Cu") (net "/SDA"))
 (segment (start 65.44375 101.1625) (end 64.29375 100.0125) (width 0.2) (layer "B.Cu") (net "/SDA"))
 (segment (start 94 98.5) (end 91.711721 100.788279) (width 0.2) (layer "B.Cu") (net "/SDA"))
 (segment (start 91.711721 100.788279) (end 73.437971 100.788279) (width 0.2) (layer "B.Cu") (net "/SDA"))
 (segment (start 73.06375 101.1625) (end 65.44375 101.1625) (width 0.2) (layer "B.Cu") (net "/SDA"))
 (segment (start 73.437971 100.788279) (end 73.06375 101.1625) (width 0.2) (layer "B.Cu") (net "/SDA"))
 (segment (start 76.5 96.348529) (end 73.986029 98.8625) (width 0.2) (layer "F.Cu") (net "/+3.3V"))
 (segment (start 89.66 91.84) (end 89 92.5) (width 0.2) (layer "F.Cu") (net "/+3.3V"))
 (segment (start 73.986029 98.8625) (end 70.52375 98.8625) (width 0.2) (layer "F.Cu") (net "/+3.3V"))
 (segment (start 70.52375 98.8625) (end 69.37375 100.0125) (width 0.2) (layer "F.Cu") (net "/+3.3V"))
 (segment (start 101.24 91.84) (end 89.66 91.84) (width 0.2) (layer "F.Cu") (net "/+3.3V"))
 (segment (start 76.5 93) (end 76.5 96.348529) (width 0.2) (layer "F.Cu") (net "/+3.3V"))
 (via (at 76.5 93) (size 0.6) (drill 0.3) (layers "F.Cu" "B.Cu") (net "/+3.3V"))
 (via (at 89 92.5) (size 0.6) (drill 0.3) (layers "F.Cu" "B.Cu") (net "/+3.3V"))
 (segment (start 89 92.5) (end 88.5 93) (width 0.2) (layer "B.Cu") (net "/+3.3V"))
 (segment (start 88.5 93) (end 76.5 93) (width 0.2) (layer "B.Cu") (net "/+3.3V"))
 (segment (start 62.22625 97) (end 59.21375 100.0125) (width 0.2) (layer "F.Cu") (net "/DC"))
 (segment (start 85.92 97) (end 80 97) (width 0.2) (layer "F.Cu") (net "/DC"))
 (segment (start 86 96.92) (end 85.92 97) (width 0.2) (layer "F.Cu") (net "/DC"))
 (segment (start 75 97) (end 62.22625 97) (width 0.2) (layer "F.Cu") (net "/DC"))
 (via (at 80 97) (size 0.6) (drill 0.3) (layers "F.Cu" "B.Cu") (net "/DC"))
 (via (at 75 97) (size 0.6) (drill 0.3) (layers "F.Cu" "B.Cu") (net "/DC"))
 (segment (start 80 97) (end 75 97) (width 0.2) (layer "B.Cu") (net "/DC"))
 (segment (start 86 99.46) (end 79.04 99.46) (width 0.2) (layer "F.Cu") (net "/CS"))
 (segment (start 72.5 96.4) (end 60.28625 96.4) (width 0.2) (layer "F.Cu") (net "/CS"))
 (segment (start 60.28625 96.4) (end 56.67375 100.0125) (width 0.2) (layer "F.Cu") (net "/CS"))
 (segment (start 79.04 99.46) (end 79 99.5) (width 0.2) (layer "F.Cu") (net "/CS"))
 (via (at 79 99.5) (size 0.6) (drill 0.3) (layers "F.Cu" "B.Cu") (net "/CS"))
 (via (at 72.5 96.4) (size 0.6) (drill 0.3) (layers "F.Cu" "B.Cu") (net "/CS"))
 (segment (start 79 99.5) (end 75.6 99.5) (width 0.2) (layer "B.Cu") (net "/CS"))
 (segment (start 75.6 99.5) (end 72.5 96.4) (width 0.2) (layer "B.Cu") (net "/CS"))
 (segment (start 69.24625 97.6) (end 66.83375 100.0125) (width 0.2) (layer "F.Cu") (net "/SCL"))
 (segment (start 70 97.6) (end 69.24625 97.6) (width 0.2) (layer "F.Cu") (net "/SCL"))
 (via (at 70 97.6) (size 0.6) (drill 0.3) (layers "F.Cu" "B.Cu") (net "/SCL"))
 (segment (start 71.80125 97.6) (end 70 97.6) (width 0.2) (layer "B.Cu") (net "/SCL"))
 (segment (start 101.24 96.92) (end 87.917895 96.92) (width 0.2) (layer "B.Cu") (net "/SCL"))
 (segment (start 86.855895 97.982) (end 81.366529 97.982) (width 0.2) (layer "B.Cu") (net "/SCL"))
 (segment (start 74.30125 100.1) (end 71.80125 97.6) (width 0.2) (layer "B.Cu") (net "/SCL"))
 (segment (start 81.366529 97.982) (end 79.248529 100.1) (width 0.2) (layer "B.Cu") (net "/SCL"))
 (segment (start 87.917895 96.92) (end 86.855895 97.982) (width 0.2) (layer "B.Cu") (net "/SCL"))
 (segment (start 79.248529 100.1) (end 74.30125 100.1) (width 0.2) (layer "B.Cu") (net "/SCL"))
 (segment (start 77.5 92.12625) (end 77.5 99) (width 0.2) (layer "F.Cu") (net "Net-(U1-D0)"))
 (segment (start 65 105.18) (end 58.42 111.76) (width 0.2) (layer "F.Cu") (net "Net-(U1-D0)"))
 (segment (start 86 86.76) (end 82.86625 86.76) (width 0.2) (layer "F.Cu") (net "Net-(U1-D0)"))
 (segment (start 77.5 99) (end 72 104.5) (width 0.2) (layer "F.Cu") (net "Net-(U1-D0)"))
 (segment (start 82.86625 86.76) (end 77.5 92.12625) (width 0.2) (layer "F.Cu") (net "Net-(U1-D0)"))
 (segment (start 72 104.5) (end 65 104.5) (width 0.2) (layer "F.Cu") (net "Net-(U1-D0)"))
 (segment (start 65 104.5) (end 65 105.18) (width 0.2) (layer "F.Cu") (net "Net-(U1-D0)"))
 (segment (start 77.9 111.33) (end 77.47 111.76) (width 0.2) (layer "F.Cu") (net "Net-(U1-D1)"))
 (segment (start 84.92237 89.3) (end 77.9 96.32237) (width 0.2) (layer "F.Cu") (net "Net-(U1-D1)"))
 (segment (start 86 89.3) (end 84.92237 89.3) (width 0.2) (layer "F.Cu") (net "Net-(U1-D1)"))
 (segment (start 77.9 96.32237) (end 77.9 111.33) (width 0.2) (layer "F.Cu") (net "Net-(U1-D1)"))
 (segment (start 96.52 102.36) (end 96.52 111.76) (width 0.2) (layer "F.Cu") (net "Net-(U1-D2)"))
 (segment (start 86 91.84) (end 96.52 102.36) (width 0.2) (layer "F.Cu") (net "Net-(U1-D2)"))
 (segment (start 97.099899 113.16) (end 98.499899 111.76) (width 0.2) (layer "F.Cu") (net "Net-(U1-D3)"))
 (segment (start 95.940101 113.16) (end 97.099899 113.16) (width 0.2) (layer "F.Cu") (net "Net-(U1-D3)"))
 (segment (start 95.12 103.5) (end 95.12 112.339899) (width 0.2) (layer "F.Cu") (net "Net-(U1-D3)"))
 (segment (start 98.499899 111.76) (end 115.57 111.76) (width 0.2) (layer "F.Cu") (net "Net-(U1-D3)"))
 (segment (start 95.12 112.339899) (end 95.940101 113.16) (width 0.2) (layer "F.Cu") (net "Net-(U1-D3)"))
 (segment (start 86 94.38) (end 95.12 103.5) (width 0.2) (layer "F.Cu") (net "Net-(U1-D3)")))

